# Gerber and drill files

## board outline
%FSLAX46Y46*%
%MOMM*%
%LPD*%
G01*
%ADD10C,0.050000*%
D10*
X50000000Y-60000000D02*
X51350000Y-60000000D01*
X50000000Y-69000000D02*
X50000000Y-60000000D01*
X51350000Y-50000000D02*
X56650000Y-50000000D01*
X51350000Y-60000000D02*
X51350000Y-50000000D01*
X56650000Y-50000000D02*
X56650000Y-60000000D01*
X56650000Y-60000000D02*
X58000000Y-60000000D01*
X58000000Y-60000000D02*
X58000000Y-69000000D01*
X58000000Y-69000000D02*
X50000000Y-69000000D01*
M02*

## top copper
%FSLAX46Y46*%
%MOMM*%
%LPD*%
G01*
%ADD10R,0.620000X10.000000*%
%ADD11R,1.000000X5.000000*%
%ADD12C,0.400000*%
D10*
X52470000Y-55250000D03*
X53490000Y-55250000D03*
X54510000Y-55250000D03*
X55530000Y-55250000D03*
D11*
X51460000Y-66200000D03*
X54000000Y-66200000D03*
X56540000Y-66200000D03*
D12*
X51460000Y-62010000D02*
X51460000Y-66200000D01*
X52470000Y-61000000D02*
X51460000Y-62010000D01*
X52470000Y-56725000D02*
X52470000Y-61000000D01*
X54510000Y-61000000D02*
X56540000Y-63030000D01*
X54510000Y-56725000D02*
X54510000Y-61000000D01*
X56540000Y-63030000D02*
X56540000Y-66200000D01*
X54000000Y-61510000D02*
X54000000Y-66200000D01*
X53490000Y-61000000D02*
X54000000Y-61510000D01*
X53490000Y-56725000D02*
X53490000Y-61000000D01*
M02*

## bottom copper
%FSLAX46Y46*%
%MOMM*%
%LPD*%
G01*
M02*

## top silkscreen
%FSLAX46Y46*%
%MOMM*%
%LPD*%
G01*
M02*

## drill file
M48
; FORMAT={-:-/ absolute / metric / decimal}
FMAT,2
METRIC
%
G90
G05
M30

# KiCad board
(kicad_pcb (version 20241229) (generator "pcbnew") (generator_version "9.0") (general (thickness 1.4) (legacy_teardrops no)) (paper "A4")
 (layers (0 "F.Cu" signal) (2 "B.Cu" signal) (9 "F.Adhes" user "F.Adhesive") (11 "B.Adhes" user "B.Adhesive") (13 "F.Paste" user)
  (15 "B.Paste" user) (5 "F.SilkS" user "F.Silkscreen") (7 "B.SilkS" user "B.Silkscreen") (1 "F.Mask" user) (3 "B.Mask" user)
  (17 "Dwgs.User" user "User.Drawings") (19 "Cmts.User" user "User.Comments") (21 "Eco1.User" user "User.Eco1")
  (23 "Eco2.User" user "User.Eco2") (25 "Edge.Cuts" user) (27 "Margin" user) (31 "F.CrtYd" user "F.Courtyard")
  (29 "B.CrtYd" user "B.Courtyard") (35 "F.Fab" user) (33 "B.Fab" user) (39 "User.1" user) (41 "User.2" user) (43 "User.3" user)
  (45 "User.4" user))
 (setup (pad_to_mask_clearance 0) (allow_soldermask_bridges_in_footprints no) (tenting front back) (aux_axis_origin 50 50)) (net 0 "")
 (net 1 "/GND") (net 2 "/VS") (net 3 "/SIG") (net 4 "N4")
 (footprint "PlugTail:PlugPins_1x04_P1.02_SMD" (layer "F.Cu") (at 54 50)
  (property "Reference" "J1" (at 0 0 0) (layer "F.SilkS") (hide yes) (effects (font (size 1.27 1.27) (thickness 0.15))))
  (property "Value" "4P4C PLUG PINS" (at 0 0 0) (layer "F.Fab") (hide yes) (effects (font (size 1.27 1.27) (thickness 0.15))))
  (pad "1" smd rect (at -1.53 5.25) (size 0.62 10) (layers "F.Cu" "F.Mask") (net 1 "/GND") (thermal_bridge_angle 45))
  (pad "2" smd rect (at -0.51 5.25) (size 0.62 10) (layers "F.Cu" "F.Mask") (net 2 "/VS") (thermal_bridge_angle 45))
  (pad "3" smd rect (at 0.51 5.25) (size 0.62 10) (layers "F.Cu" "F.Mask") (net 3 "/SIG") (thermal_bridge_angle 45))
  (pad "4" smd rect (at 1.53 5.25) (size 0.62 10) (layers "F.Cu" "F.Mask") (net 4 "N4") (thermal_bridge_angle 45)))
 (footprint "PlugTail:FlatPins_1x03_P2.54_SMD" (layer "F.Cu") (at 54 66.2)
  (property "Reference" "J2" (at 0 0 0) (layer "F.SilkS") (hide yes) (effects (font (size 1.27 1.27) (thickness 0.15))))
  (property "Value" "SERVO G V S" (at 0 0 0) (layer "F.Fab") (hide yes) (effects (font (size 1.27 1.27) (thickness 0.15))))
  (pad "1" smd rect (at -2.54 0) (size 1 5) (layers "F.Cu" "F.Mask") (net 1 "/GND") (thermal_bridge_angle 45))
  (pad "2" smd rect (at 0 0) (size 1 5) (layers "F.Cu" "F.Mask") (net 2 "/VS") (thermal_bridge_angle 45))
  (pad "3" smd rect (at 2.54 0) (size 1 5) (layers "F.Cu" "F.Mask") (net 3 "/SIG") (thermal_bridge_angle 45)))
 (gr_line (start 50 60) (end 51.35 60) (stroke (width 0.05) (type default)) (layer "Edge.Cuts"))
 (gr_line (start 50 69) (end 50 60) (stroke (width 0.05) (type default)) (layer "Edge.Cuts"))
 (gr_line (start 51.35 50) (end 56.65 50) (stroke (width 0.05) (type default)) (layer "Edge.Cuts"))
 (gr_line (start 51.35 60) (end 51.35 50) (stroke (width 0.05) (type default)) (layer "Edge.Cuts"))
 (gr_line (start 56.65 50) (end 56.65 60) (stroke (width 0.05) (type default)) (layer "Edge.Cuts"))
 (gr_line (start 56.65 60) (end 58 60) (stroke (width 0.05) (type default)) (layer "Edge.Cuts"))
 (gr_line (start 58 60) (end 58 69) (stroke (width 0.05) (type default)) (layer "Edge.Cuts"))
 (gr_line (start 58 69) (end 50 69) (stroke (width 0.05) (type default)) (layer "Edge.Cuts"))
 (segment (start 51.46 62.01) (end 51.46 66.2) (width 0.4) (layer "F.Cu") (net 1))
 (segment (start 52.47 61) (end 51.46 62.01) (width 0.4) (layer "F.Cu") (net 1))
 (segment (start 52.47 56.725) (end 52.47 61) (width 0.4) (layer "F.Cu") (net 1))
 (segment (start 54.51 61) (end 56.54 63.03) (width 0.4) (layer "F.Cu") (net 3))
 (segment (start 54.51 56.725) (end 54.51 61) (width 0.4) (layer "F.Cu") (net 3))
 (segment (start 56.54 63.03) (end 56.54 66.2) (width 0.4) (layer "F.Cu") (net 3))
 (segment (start 54 61.51) (end 54 66.2) (width 0.4) (layer "F.Cu") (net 2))
 (segment (start 53.49 61) (end 54 61.51) (width 0.4) (layer "F.Cu") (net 2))
 (segment (start 53.49 56.725) (end 53.49 61) (width 0.4) (layer "F.Cu") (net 2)))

